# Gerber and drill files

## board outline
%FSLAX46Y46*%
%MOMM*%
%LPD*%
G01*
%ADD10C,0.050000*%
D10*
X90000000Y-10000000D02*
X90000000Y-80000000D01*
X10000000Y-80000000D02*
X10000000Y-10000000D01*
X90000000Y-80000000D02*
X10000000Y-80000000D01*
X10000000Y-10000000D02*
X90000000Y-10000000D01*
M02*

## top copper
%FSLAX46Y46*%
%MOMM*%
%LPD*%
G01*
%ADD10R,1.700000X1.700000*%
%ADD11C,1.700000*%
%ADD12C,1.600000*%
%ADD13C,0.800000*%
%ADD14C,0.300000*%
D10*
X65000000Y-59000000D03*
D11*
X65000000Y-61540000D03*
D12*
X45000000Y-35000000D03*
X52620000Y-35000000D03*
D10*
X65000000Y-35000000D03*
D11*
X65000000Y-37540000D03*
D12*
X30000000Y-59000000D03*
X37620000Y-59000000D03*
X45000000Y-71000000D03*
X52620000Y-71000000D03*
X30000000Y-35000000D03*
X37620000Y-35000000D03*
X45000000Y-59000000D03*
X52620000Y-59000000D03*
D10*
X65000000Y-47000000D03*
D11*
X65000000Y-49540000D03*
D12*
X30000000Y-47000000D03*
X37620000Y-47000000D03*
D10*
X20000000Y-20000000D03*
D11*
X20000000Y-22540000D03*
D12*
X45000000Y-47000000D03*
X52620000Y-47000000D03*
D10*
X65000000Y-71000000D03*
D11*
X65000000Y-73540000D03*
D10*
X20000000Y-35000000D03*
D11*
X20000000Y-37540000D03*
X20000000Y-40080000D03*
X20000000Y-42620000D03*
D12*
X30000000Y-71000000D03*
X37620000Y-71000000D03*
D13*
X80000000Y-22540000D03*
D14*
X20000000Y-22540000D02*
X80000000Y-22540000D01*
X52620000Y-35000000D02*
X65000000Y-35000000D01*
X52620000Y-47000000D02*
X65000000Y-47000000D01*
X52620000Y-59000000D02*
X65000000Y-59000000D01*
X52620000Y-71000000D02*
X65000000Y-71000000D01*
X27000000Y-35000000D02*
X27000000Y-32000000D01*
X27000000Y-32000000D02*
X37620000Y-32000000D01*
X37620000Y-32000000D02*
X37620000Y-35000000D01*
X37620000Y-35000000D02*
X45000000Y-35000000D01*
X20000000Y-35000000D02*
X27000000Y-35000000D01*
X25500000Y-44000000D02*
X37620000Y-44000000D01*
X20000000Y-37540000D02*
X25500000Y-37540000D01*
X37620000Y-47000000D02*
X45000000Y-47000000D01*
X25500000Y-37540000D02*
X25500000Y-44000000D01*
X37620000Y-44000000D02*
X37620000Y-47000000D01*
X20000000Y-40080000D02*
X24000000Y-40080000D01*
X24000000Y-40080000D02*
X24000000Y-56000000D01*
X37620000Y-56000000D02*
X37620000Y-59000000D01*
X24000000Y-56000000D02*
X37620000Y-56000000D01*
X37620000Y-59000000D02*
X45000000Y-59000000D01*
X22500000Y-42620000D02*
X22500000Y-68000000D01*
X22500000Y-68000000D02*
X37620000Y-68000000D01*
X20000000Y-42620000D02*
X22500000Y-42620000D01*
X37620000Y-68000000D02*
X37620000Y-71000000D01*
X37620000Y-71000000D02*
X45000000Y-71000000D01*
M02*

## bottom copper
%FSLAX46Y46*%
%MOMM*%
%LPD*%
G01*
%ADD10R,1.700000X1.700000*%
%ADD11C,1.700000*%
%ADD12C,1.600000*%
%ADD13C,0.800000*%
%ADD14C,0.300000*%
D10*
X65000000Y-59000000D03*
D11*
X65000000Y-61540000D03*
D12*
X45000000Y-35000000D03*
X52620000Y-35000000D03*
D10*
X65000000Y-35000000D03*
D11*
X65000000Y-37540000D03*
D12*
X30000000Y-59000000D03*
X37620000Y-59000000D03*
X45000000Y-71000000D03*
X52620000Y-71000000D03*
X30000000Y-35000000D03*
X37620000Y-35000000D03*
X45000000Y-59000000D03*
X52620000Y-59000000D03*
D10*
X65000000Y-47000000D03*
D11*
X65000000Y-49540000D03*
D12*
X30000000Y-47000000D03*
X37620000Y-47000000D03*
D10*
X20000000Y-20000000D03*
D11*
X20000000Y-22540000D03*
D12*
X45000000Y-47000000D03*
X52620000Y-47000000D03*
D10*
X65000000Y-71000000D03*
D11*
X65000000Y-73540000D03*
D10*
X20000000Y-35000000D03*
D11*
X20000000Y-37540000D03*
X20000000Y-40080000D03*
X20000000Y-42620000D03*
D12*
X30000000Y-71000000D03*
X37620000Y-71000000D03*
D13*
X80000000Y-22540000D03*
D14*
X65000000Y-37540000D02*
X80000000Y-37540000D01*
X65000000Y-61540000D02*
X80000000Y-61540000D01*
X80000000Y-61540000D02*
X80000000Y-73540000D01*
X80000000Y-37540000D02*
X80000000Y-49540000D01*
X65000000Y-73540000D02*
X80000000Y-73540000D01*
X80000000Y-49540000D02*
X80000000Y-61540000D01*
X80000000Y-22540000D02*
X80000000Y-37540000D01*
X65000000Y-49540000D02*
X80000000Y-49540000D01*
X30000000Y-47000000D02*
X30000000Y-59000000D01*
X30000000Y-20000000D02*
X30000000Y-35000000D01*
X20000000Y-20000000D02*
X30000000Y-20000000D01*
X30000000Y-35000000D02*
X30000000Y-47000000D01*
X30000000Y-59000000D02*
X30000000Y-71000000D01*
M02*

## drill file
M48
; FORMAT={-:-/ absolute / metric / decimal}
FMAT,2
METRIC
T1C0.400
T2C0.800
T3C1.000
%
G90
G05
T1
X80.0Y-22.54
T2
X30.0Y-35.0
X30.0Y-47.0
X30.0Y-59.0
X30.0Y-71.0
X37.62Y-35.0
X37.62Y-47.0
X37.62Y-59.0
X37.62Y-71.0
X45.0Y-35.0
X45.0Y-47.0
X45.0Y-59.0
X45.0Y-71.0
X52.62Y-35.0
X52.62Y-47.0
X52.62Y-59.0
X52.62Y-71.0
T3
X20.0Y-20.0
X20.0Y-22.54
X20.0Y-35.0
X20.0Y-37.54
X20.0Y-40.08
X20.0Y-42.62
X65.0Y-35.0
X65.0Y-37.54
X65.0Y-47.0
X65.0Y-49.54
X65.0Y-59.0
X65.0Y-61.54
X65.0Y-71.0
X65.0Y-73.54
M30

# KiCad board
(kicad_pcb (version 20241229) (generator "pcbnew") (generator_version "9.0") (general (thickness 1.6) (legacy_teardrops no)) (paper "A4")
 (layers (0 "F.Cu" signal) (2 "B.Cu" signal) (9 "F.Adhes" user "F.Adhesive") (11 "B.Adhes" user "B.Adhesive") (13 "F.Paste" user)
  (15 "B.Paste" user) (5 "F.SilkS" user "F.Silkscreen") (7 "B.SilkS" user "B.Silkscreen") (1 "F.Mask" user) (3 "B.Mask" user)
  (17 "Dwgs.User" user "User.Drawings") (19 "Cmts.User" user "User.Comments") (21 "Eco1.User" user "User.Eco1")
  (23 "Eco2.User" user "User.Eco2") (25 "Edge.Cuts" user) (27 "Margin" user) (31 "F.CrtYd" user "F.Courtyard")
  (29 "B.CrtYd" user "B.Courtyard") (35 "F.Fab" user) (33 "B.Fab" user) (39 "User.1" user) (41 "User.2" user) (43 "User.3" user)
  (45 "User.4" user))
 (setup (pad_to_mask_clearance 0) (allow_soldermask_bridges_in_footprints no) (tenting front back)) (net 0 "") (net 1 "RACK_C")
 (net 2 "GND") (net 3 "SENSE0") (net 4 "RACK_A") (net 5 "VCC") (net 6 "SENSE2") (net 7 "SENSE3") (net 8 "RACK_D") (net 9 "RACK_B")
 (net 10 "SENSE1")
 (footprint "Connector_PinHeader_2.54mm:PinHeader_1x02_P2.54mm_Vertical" (layer "F.Cu") (at 65 59)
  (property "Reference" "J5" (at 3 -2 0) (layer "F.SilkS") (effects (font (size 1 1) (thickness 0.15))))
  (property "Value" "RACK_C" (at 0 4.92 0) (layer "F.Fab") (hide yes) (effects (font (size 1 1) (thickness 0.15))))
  (pad "1" thru_hole rect (at 0 0) (size 1.7 1.7) (drill 1) (layers "*.Cu" "*.Mask") (remove_unused_layers no) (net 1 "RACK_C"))
  (pad "2" thru_hole circle (at 0 2.54) (size 1.7 1.7) (drill 1) (layers "*.Cu" "*.Mask") (remove_unused_layers no) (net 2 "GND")))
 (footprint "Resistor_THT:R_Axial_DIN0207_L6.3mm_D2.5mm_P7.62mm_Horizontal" (layer "F.Cu") (at 45 35)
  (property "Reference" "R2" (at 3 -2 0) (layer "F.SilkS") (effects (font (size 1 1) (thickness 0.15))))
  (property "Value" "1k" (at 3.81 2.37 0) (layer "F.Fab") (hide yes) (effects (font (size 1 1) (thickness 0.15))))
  (pad "1" thru_hole circle (at 0 0) (size 1.6 1.6) (drill 0.8) (layers "*.Cu" "*.Mask") (remove_unused_layers no) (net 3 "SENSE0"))
  (pad "2" thru_hole circle (at 7.62 0) (size 1.6 1.6) (drill 0.8) (layers "*.Cu" "*.Mask") (remove_unused_layers no) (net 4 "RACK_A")))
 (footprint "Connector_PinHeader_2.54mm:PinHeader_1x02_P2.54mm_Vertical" (layer "F.Cu") (at 65 35)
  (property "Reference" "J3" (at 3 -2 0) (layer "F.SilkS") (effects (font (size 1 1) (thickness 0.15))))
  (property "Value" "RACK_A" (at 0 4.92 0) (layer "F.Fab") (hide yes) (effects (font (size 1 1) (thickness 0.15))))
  (pad "1" thru_hole rect (at 0 0) (size 1.7 1.7) (drill 1) (layers "*.Cu" "*.Mask") (remove_unused_layers no) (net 4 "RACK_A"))
  (pad "2" thru_hole circle (at 0 2.54) (size 1.7 1.7) (drill 1) (layers "*.Cu" "*.Mask") (remove_unused_layers no) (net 2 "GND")))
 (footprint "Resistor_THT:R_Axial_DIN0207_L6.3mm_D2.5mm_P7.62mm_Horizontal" (layer "F.Cu") (at 30 59)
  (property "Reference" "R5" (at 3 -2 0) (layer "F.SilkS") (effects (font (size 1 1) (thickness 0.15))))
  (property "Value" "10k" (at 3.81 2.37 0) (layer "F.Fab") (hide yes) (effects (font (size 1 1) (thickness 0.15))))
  (pad "1" thru_hole circle (at 0 0) (size 1.6 1.6) (drill 0.8) (layers "*.Cu" "*.Mask") (remove_unused_layers no) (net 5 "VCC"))
  (pad "2" thru_hole circle (at 7.62 0) (size 1.6 1.6) (drill 0.8) (layers "*.Cu" "*.Mask") (remove_unused_layers no) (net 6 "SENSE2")))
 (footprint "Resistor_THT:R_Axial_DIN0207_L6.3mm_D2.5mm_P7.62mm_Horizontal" (layer "F.Cu") (at 45 71)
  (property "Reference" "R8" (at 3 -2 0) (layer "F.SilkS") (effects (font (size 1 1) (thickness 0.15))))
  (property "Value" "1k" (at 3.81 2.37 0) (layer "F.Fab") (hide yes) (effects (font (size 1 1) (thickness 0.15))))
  (pad "1" thru_hole circle (at 0 0) (size 1.6 1.6) (drill 0.8) (layers "*.Cu" "*.Mask") (remove_unused_layers no) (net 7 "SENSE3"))
  (pad "2" thru_hole circle (at 7.62 0) (size 1.6 1.6) (drill 0.8) (layers "*.Cu" "*.Mask") (remove_unused_layers no) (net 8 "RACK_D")))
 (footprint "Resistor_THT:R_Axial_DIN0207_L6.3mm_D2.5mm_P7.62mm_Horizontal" (layer "F.Cu") (at 30 35)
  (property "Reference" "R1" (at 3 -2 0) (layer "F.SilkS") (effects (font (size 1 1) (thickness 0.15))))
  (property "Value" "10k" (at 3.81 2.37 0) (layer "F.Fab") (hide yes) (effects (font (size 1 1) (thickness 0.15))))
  (pad "1" thru_hole circle (at 0 0) (size 1.6 1.6) (drill 0.8) (layers "*.Cu" "*.Mask") (remove_unused_layers no) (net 5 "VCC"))
  (pad "2" thru_hole circle (at 7.62 0) (size 1.6 1.6) (drill 0.8) (layers "*.Cu" "*.Mask") (remove_unused_layers no) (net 3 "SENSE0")))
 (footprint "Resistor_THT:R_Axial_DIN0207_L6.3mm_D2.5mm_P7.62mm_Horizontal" (layer "F.Cu") (at 45 59)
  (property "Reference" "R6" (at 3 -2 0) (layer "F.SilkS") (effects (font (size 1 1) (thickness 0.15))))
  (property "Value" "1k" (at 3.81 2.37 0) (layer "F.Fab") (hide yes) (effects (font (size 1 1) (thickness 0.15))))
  (pad "1" thru_hole circle (at 0 0) (size 1.6 1.6) (drill 0.8) (layers "*.Cu" "*.Mask") (remove_unused_layers no) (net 6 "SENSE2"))
  (pad "2" thru_hole circle (at 7.62 0) (size 1.6 1.6) (drill 0.8) (layers "*.Cu" "*.Mask") (remove_unused_layers no) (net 1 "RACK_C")))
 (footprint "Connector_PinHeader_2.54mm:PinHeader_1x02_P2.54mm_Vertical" (layer "F.Cu") (at 65 47)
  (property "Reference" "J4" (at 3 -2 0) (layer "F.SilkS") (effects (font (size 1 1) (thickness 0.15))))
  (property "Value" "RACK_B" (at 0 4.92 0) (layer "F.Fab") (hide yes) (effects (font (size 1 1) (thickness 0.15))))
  (pad "1" thru_hole rect (at 0 0) (size 1.7 1.7) (drill 1) (layers "*.Cu" "*.Mask") (remove_unused_layers no) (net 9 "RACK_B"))
  (pad "2" thru_hole circle (at 0 2.54) (size 1.7 1.7) (drill 1) (layers "*.Cu" "*.Mask") (remove_unused_layers no) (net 2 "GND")))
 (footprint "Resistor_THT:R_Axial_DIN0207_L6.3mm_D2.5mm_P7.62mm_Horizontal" (layer "F.Cu") (at 30 47)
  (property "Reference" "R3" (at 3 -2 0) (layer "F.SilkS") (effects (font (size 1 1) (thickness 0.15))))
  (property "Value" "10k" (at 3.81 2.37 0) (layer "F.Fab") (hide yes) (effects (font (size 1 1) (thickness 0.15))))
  (pad "1" thru_hole circle (at 0 0) (size 1.6 1.6) (drill 0.8) (layers "*.Cu" "*.Mask") (remove_unused_layers no) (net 5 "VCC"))
  (pad "2" thru_hole circle (at 7.62 0) (size 1.6 1.6) (drill 0.8) (layers "*.Cu" "*.Mask") (remove_unused_layers no) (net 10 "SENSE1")))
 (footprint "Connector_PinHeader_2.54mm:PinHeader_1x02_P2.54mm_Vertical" (layer "F.Cu") (at 20 20)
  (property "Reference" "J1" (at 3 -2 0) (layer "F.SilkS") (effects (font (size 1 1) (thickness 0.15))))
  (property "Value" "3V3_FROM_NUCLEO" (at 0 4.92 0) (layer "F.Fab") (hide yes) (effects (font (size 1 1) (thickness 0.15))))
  (pad "1" thru_hole rect (at 0 0) (size 1.7 1.7) (drill 1) (layers "*.Cu" "*.Mask") (remove_unused_layers no) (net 5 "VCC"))
  (pad "2" thru_hole circle (at 0 2.54) (size 1.7 1.7) (drill 1) (layers "*.Cu" "*.Mask") (remove_unused_layers no) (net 2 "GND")))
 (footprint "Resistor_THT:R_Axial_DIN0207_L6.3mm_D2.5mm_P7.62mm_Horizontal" (layer "F.Cu") (at 45 47)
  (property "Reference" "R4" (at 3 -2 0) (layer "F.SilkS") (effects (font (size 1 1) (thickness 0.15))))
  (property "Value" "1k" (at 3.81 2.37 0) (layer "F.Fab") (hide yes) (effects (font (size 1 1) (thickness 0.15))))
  (pad "1" thru_hole circle (at 0 0) (size 1.6 1.6) (drill 0.8) (layers "*.Cu" "*.Mask") (remove_unused_layers no) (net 10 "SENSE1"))
  (pad "2" thru_hole circle (at 7.62 0) (size 1.6 1.6) (drill 0.8) (layers "*.Cu" "*.Mask") (remove_unused_layers no) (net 9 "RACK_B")))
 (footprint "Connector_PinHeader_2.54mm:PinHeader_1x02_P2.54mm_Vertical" (layer "F.Cu") (at 65 71)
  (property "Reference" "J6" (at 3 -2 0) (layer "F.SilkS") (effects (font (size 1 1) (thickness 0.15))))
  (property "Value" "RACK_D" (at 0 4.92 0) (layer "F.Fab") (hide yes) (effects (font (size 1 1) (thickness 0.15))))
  (pad "1" thru_hole rect (at 0 0) (size 1.7 1.7) (drill 1) (layers "*.Cu" "*.Mask") (remove_unused_layers no) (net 8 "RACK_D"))
  (pad "2" thru_hole circle (at 0 2.54) (size 1.7 1.7) (drill 1) (layers "*.Cu" "*.Mask") (remove_unused_layers no) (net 2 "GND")))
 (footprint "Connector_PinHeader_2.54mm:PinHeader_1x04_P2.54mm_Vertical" (layer "F.Cu") (at 20 35)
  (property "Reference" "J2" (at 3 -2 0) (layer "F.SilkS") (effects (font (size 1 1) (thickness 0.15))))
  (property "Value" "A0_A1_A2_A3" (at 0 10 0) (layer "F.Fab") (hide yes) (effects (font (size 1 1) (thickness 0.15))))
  (pad "1" thru_hole rect (at 0 0) (size 1.7 1.7) (drill 1) (layers "*.Cu" "*.Mask") (remove_unused_layers no) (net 3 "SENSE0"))
  (pad "2" thru_hole circle (at 0 2.54) (size 1.7 1.7) (drill 1) (layers "*.Cu" "*.Mask") (remove_unused_layers no) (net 10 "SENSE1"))
  (pad "3" thru_hole circle (at 0 5.08) (size 1.7 1.7) (drill 1) (layers "*.Cu" "*.Mask") (remove_unused_layers no) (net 6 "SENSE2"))
  (pad "4" thru_hole circle (at 0 7.62) (size 1.7 1.7) (drill 1) (layers "*.Cu" "*.Mask") (remove_unused_layers no) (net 7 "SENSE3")))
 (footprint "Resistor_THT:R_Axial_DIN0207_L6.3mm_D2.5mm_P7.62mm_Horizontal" (layer "F.Cu") (at 30 71)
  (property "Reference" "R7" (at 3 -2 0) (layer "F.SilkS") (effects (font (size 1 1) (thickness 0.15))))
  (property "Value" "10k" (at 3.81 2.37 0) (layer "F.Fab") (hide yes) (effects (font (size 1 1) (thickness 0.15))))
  (pad "1" thru_hole circle (at 0 0) (size 1.6 1.6) (drill 0.8) (layers "*.Cu" "*.Mask") (remove_unused_layers no) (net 5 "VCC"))
  (pad "2" thru_hole circle (at 7.62 0) (size 1.6 1.6) (drill 0.8) (layers "*.Cu" "*.Mask") (remove_unused_layers no) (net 7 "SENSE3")))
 (gr_line (start 90 10) (end 90 80) (stroke (width 0.05) (type default)) (layer "Edge.Cuts"))
 (gr_line (start 10 80) (end 10 10) (stroke (width 0.05) (type default)) (layer "Edge.Cuts"))
 (gr_line (start 90 80) (end 10 80) (stroke (width 0.05) (type default)) (layer "Edge.Cuts"))
 (gr_line (start 10 10) (end 90 10) (stroke (width 0.05) (type default)) (layer "Edge.Cuts"))
 (segment (start 20 22.54) (end 80 22.54) (width 0.3) (layer "F.Cu") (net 2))
 (via (at 80 22.54) (size 0.8) (drill 0.4) (layers "F.Cu" "B.Cu") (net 2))
 (segment (start 65 37.54) (end 80 37.54) (width 0.3) (layer "B.Cu") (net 2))
 (segment (start 65 61.54) (end 80 61.54) (width 0.3) (layer "B.Cu") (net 2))
 (segment (start 80 61.54) (end 80 73.54) (width 0.3) (layer "B.Cu") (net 2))
 (segment (start 80 37.54) (end 80 49.54) (width 0.3) (layer "B.Cu") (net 2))
 (segment (start 65 73.54) (end 80 73.54) (width 0.3) (layer "B.Cu") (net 2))
 (segment (start 80 49.54) (end 80 61.54) (width 0.3) (layer "B.Cu") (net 2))
 (segment (start 80 22.54) (end 80 37.54) (width 0.3) (layer "B.Cu") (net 2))
 (segment (start 65 49.54) (end 80 49.54) (width 0.3) (layer "B.Cu") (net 2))
 (segment (start 52.62 35) (end 65 35) (width 0.3) (layer "F.Cu") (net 4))
 (segment (start 52.62 47) (end 65 47) (width 0.3) (layer "F.Cu") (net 9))
 (segment (start 52.62 59) (end 65 59) (width 0.3) (layer "F.Cu") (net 1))
 (segment (start 52.62 71) (end 65 71) (width 0.3) (layer "F.Cu") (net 8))
 (segment (start 27 35) (end 27 32) (width 0.3) (layer "F.Cu") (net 3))
 (segment (start 27 32) (end 37.62 32) (width 0.3) (layer "F.Cu") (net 3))
 (segment (start 37.62 32) (end 37.62 35) (width 0.3) (layer "F.Cu") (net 3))
 (segment (start 37.62 35) (end 45 35) (width 0.3) (layer "F.Cu") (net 3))
 (segment (start 20 35) (end 27 35) (width 0.3) (layer "F.Cu") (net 3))
 (segment (start 25.5 44) (end 37.62 44) (width 0.3) (layer "F.Cu") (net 10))
 (segment (start 20 37.54) (end 25.5 37.54) (width 0.3) (layer "F.Cu") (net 10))
 (segment (start 37.62 47) (end 45 47) (width 0.3) (layer "F.Cu") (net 10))
 (segment (start 25.5 37.54) (end 25.5 44) (width 0.3) (layer "F.Cu") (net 10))
 (segment (start 37.62 44) (end 37.62 47) (width 0.3) (layer "F.Cu") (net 10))
 (segment (start 20 40.08) (end 24 40.08) (width 0.3) (layer "F.Cu") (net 6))
 (segment (start 24 40.08) (end 24 56) (width 0.3) (layer "F.Cu") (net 6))
 (segment (start 37.62 56) (end 37.62 59) (width 0.3) (layer "F.Cu") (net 6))
 (segment (start 24 56) (end 37.62 56) (width 0.3) (layer "F.Cu") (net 6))
 (segment (start 37.62 59) (end 45 59) (width 0.3) (layer "F.Cu") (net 6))
 (segment (start 22.5 42.62) (end 22.5 68) (width 0.3) (layer "F.Cu") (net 7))
 (segment (start 22.5 68) (end 37.62 68) (width 0.3) (layer "F.Cu") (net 7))
 (segment (start 20 42.62) (end 22.5 42.62) (width 0.3) (layer "F.Cu") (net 7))
 (segment (start 37.62 68) (end 37.62 71) (width 0.3) (layer "F.Cu") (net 7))
 (segment (start 37.62 71) (end 45 71) (width 0.3) (layer "F.Cu") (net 7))
 (segment (start 30 47) (end 30 59) (width 0.3) (layer "B.Cu") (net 5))
 (segment (start 30 20) (end 30 35) (width 0.3) (layer "B.Cu") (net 5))
 (segment (start 20 20) (end 30 20) (width 0.3) (layer "B.Cu") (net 5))
 (segment (start 30 35) (end 30 47) (width 0.3) (layer "B.Cu") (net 5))
 (segment (start 30 59) (end 30 71) (width 0.3) (layer "B.Cu") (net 5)))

